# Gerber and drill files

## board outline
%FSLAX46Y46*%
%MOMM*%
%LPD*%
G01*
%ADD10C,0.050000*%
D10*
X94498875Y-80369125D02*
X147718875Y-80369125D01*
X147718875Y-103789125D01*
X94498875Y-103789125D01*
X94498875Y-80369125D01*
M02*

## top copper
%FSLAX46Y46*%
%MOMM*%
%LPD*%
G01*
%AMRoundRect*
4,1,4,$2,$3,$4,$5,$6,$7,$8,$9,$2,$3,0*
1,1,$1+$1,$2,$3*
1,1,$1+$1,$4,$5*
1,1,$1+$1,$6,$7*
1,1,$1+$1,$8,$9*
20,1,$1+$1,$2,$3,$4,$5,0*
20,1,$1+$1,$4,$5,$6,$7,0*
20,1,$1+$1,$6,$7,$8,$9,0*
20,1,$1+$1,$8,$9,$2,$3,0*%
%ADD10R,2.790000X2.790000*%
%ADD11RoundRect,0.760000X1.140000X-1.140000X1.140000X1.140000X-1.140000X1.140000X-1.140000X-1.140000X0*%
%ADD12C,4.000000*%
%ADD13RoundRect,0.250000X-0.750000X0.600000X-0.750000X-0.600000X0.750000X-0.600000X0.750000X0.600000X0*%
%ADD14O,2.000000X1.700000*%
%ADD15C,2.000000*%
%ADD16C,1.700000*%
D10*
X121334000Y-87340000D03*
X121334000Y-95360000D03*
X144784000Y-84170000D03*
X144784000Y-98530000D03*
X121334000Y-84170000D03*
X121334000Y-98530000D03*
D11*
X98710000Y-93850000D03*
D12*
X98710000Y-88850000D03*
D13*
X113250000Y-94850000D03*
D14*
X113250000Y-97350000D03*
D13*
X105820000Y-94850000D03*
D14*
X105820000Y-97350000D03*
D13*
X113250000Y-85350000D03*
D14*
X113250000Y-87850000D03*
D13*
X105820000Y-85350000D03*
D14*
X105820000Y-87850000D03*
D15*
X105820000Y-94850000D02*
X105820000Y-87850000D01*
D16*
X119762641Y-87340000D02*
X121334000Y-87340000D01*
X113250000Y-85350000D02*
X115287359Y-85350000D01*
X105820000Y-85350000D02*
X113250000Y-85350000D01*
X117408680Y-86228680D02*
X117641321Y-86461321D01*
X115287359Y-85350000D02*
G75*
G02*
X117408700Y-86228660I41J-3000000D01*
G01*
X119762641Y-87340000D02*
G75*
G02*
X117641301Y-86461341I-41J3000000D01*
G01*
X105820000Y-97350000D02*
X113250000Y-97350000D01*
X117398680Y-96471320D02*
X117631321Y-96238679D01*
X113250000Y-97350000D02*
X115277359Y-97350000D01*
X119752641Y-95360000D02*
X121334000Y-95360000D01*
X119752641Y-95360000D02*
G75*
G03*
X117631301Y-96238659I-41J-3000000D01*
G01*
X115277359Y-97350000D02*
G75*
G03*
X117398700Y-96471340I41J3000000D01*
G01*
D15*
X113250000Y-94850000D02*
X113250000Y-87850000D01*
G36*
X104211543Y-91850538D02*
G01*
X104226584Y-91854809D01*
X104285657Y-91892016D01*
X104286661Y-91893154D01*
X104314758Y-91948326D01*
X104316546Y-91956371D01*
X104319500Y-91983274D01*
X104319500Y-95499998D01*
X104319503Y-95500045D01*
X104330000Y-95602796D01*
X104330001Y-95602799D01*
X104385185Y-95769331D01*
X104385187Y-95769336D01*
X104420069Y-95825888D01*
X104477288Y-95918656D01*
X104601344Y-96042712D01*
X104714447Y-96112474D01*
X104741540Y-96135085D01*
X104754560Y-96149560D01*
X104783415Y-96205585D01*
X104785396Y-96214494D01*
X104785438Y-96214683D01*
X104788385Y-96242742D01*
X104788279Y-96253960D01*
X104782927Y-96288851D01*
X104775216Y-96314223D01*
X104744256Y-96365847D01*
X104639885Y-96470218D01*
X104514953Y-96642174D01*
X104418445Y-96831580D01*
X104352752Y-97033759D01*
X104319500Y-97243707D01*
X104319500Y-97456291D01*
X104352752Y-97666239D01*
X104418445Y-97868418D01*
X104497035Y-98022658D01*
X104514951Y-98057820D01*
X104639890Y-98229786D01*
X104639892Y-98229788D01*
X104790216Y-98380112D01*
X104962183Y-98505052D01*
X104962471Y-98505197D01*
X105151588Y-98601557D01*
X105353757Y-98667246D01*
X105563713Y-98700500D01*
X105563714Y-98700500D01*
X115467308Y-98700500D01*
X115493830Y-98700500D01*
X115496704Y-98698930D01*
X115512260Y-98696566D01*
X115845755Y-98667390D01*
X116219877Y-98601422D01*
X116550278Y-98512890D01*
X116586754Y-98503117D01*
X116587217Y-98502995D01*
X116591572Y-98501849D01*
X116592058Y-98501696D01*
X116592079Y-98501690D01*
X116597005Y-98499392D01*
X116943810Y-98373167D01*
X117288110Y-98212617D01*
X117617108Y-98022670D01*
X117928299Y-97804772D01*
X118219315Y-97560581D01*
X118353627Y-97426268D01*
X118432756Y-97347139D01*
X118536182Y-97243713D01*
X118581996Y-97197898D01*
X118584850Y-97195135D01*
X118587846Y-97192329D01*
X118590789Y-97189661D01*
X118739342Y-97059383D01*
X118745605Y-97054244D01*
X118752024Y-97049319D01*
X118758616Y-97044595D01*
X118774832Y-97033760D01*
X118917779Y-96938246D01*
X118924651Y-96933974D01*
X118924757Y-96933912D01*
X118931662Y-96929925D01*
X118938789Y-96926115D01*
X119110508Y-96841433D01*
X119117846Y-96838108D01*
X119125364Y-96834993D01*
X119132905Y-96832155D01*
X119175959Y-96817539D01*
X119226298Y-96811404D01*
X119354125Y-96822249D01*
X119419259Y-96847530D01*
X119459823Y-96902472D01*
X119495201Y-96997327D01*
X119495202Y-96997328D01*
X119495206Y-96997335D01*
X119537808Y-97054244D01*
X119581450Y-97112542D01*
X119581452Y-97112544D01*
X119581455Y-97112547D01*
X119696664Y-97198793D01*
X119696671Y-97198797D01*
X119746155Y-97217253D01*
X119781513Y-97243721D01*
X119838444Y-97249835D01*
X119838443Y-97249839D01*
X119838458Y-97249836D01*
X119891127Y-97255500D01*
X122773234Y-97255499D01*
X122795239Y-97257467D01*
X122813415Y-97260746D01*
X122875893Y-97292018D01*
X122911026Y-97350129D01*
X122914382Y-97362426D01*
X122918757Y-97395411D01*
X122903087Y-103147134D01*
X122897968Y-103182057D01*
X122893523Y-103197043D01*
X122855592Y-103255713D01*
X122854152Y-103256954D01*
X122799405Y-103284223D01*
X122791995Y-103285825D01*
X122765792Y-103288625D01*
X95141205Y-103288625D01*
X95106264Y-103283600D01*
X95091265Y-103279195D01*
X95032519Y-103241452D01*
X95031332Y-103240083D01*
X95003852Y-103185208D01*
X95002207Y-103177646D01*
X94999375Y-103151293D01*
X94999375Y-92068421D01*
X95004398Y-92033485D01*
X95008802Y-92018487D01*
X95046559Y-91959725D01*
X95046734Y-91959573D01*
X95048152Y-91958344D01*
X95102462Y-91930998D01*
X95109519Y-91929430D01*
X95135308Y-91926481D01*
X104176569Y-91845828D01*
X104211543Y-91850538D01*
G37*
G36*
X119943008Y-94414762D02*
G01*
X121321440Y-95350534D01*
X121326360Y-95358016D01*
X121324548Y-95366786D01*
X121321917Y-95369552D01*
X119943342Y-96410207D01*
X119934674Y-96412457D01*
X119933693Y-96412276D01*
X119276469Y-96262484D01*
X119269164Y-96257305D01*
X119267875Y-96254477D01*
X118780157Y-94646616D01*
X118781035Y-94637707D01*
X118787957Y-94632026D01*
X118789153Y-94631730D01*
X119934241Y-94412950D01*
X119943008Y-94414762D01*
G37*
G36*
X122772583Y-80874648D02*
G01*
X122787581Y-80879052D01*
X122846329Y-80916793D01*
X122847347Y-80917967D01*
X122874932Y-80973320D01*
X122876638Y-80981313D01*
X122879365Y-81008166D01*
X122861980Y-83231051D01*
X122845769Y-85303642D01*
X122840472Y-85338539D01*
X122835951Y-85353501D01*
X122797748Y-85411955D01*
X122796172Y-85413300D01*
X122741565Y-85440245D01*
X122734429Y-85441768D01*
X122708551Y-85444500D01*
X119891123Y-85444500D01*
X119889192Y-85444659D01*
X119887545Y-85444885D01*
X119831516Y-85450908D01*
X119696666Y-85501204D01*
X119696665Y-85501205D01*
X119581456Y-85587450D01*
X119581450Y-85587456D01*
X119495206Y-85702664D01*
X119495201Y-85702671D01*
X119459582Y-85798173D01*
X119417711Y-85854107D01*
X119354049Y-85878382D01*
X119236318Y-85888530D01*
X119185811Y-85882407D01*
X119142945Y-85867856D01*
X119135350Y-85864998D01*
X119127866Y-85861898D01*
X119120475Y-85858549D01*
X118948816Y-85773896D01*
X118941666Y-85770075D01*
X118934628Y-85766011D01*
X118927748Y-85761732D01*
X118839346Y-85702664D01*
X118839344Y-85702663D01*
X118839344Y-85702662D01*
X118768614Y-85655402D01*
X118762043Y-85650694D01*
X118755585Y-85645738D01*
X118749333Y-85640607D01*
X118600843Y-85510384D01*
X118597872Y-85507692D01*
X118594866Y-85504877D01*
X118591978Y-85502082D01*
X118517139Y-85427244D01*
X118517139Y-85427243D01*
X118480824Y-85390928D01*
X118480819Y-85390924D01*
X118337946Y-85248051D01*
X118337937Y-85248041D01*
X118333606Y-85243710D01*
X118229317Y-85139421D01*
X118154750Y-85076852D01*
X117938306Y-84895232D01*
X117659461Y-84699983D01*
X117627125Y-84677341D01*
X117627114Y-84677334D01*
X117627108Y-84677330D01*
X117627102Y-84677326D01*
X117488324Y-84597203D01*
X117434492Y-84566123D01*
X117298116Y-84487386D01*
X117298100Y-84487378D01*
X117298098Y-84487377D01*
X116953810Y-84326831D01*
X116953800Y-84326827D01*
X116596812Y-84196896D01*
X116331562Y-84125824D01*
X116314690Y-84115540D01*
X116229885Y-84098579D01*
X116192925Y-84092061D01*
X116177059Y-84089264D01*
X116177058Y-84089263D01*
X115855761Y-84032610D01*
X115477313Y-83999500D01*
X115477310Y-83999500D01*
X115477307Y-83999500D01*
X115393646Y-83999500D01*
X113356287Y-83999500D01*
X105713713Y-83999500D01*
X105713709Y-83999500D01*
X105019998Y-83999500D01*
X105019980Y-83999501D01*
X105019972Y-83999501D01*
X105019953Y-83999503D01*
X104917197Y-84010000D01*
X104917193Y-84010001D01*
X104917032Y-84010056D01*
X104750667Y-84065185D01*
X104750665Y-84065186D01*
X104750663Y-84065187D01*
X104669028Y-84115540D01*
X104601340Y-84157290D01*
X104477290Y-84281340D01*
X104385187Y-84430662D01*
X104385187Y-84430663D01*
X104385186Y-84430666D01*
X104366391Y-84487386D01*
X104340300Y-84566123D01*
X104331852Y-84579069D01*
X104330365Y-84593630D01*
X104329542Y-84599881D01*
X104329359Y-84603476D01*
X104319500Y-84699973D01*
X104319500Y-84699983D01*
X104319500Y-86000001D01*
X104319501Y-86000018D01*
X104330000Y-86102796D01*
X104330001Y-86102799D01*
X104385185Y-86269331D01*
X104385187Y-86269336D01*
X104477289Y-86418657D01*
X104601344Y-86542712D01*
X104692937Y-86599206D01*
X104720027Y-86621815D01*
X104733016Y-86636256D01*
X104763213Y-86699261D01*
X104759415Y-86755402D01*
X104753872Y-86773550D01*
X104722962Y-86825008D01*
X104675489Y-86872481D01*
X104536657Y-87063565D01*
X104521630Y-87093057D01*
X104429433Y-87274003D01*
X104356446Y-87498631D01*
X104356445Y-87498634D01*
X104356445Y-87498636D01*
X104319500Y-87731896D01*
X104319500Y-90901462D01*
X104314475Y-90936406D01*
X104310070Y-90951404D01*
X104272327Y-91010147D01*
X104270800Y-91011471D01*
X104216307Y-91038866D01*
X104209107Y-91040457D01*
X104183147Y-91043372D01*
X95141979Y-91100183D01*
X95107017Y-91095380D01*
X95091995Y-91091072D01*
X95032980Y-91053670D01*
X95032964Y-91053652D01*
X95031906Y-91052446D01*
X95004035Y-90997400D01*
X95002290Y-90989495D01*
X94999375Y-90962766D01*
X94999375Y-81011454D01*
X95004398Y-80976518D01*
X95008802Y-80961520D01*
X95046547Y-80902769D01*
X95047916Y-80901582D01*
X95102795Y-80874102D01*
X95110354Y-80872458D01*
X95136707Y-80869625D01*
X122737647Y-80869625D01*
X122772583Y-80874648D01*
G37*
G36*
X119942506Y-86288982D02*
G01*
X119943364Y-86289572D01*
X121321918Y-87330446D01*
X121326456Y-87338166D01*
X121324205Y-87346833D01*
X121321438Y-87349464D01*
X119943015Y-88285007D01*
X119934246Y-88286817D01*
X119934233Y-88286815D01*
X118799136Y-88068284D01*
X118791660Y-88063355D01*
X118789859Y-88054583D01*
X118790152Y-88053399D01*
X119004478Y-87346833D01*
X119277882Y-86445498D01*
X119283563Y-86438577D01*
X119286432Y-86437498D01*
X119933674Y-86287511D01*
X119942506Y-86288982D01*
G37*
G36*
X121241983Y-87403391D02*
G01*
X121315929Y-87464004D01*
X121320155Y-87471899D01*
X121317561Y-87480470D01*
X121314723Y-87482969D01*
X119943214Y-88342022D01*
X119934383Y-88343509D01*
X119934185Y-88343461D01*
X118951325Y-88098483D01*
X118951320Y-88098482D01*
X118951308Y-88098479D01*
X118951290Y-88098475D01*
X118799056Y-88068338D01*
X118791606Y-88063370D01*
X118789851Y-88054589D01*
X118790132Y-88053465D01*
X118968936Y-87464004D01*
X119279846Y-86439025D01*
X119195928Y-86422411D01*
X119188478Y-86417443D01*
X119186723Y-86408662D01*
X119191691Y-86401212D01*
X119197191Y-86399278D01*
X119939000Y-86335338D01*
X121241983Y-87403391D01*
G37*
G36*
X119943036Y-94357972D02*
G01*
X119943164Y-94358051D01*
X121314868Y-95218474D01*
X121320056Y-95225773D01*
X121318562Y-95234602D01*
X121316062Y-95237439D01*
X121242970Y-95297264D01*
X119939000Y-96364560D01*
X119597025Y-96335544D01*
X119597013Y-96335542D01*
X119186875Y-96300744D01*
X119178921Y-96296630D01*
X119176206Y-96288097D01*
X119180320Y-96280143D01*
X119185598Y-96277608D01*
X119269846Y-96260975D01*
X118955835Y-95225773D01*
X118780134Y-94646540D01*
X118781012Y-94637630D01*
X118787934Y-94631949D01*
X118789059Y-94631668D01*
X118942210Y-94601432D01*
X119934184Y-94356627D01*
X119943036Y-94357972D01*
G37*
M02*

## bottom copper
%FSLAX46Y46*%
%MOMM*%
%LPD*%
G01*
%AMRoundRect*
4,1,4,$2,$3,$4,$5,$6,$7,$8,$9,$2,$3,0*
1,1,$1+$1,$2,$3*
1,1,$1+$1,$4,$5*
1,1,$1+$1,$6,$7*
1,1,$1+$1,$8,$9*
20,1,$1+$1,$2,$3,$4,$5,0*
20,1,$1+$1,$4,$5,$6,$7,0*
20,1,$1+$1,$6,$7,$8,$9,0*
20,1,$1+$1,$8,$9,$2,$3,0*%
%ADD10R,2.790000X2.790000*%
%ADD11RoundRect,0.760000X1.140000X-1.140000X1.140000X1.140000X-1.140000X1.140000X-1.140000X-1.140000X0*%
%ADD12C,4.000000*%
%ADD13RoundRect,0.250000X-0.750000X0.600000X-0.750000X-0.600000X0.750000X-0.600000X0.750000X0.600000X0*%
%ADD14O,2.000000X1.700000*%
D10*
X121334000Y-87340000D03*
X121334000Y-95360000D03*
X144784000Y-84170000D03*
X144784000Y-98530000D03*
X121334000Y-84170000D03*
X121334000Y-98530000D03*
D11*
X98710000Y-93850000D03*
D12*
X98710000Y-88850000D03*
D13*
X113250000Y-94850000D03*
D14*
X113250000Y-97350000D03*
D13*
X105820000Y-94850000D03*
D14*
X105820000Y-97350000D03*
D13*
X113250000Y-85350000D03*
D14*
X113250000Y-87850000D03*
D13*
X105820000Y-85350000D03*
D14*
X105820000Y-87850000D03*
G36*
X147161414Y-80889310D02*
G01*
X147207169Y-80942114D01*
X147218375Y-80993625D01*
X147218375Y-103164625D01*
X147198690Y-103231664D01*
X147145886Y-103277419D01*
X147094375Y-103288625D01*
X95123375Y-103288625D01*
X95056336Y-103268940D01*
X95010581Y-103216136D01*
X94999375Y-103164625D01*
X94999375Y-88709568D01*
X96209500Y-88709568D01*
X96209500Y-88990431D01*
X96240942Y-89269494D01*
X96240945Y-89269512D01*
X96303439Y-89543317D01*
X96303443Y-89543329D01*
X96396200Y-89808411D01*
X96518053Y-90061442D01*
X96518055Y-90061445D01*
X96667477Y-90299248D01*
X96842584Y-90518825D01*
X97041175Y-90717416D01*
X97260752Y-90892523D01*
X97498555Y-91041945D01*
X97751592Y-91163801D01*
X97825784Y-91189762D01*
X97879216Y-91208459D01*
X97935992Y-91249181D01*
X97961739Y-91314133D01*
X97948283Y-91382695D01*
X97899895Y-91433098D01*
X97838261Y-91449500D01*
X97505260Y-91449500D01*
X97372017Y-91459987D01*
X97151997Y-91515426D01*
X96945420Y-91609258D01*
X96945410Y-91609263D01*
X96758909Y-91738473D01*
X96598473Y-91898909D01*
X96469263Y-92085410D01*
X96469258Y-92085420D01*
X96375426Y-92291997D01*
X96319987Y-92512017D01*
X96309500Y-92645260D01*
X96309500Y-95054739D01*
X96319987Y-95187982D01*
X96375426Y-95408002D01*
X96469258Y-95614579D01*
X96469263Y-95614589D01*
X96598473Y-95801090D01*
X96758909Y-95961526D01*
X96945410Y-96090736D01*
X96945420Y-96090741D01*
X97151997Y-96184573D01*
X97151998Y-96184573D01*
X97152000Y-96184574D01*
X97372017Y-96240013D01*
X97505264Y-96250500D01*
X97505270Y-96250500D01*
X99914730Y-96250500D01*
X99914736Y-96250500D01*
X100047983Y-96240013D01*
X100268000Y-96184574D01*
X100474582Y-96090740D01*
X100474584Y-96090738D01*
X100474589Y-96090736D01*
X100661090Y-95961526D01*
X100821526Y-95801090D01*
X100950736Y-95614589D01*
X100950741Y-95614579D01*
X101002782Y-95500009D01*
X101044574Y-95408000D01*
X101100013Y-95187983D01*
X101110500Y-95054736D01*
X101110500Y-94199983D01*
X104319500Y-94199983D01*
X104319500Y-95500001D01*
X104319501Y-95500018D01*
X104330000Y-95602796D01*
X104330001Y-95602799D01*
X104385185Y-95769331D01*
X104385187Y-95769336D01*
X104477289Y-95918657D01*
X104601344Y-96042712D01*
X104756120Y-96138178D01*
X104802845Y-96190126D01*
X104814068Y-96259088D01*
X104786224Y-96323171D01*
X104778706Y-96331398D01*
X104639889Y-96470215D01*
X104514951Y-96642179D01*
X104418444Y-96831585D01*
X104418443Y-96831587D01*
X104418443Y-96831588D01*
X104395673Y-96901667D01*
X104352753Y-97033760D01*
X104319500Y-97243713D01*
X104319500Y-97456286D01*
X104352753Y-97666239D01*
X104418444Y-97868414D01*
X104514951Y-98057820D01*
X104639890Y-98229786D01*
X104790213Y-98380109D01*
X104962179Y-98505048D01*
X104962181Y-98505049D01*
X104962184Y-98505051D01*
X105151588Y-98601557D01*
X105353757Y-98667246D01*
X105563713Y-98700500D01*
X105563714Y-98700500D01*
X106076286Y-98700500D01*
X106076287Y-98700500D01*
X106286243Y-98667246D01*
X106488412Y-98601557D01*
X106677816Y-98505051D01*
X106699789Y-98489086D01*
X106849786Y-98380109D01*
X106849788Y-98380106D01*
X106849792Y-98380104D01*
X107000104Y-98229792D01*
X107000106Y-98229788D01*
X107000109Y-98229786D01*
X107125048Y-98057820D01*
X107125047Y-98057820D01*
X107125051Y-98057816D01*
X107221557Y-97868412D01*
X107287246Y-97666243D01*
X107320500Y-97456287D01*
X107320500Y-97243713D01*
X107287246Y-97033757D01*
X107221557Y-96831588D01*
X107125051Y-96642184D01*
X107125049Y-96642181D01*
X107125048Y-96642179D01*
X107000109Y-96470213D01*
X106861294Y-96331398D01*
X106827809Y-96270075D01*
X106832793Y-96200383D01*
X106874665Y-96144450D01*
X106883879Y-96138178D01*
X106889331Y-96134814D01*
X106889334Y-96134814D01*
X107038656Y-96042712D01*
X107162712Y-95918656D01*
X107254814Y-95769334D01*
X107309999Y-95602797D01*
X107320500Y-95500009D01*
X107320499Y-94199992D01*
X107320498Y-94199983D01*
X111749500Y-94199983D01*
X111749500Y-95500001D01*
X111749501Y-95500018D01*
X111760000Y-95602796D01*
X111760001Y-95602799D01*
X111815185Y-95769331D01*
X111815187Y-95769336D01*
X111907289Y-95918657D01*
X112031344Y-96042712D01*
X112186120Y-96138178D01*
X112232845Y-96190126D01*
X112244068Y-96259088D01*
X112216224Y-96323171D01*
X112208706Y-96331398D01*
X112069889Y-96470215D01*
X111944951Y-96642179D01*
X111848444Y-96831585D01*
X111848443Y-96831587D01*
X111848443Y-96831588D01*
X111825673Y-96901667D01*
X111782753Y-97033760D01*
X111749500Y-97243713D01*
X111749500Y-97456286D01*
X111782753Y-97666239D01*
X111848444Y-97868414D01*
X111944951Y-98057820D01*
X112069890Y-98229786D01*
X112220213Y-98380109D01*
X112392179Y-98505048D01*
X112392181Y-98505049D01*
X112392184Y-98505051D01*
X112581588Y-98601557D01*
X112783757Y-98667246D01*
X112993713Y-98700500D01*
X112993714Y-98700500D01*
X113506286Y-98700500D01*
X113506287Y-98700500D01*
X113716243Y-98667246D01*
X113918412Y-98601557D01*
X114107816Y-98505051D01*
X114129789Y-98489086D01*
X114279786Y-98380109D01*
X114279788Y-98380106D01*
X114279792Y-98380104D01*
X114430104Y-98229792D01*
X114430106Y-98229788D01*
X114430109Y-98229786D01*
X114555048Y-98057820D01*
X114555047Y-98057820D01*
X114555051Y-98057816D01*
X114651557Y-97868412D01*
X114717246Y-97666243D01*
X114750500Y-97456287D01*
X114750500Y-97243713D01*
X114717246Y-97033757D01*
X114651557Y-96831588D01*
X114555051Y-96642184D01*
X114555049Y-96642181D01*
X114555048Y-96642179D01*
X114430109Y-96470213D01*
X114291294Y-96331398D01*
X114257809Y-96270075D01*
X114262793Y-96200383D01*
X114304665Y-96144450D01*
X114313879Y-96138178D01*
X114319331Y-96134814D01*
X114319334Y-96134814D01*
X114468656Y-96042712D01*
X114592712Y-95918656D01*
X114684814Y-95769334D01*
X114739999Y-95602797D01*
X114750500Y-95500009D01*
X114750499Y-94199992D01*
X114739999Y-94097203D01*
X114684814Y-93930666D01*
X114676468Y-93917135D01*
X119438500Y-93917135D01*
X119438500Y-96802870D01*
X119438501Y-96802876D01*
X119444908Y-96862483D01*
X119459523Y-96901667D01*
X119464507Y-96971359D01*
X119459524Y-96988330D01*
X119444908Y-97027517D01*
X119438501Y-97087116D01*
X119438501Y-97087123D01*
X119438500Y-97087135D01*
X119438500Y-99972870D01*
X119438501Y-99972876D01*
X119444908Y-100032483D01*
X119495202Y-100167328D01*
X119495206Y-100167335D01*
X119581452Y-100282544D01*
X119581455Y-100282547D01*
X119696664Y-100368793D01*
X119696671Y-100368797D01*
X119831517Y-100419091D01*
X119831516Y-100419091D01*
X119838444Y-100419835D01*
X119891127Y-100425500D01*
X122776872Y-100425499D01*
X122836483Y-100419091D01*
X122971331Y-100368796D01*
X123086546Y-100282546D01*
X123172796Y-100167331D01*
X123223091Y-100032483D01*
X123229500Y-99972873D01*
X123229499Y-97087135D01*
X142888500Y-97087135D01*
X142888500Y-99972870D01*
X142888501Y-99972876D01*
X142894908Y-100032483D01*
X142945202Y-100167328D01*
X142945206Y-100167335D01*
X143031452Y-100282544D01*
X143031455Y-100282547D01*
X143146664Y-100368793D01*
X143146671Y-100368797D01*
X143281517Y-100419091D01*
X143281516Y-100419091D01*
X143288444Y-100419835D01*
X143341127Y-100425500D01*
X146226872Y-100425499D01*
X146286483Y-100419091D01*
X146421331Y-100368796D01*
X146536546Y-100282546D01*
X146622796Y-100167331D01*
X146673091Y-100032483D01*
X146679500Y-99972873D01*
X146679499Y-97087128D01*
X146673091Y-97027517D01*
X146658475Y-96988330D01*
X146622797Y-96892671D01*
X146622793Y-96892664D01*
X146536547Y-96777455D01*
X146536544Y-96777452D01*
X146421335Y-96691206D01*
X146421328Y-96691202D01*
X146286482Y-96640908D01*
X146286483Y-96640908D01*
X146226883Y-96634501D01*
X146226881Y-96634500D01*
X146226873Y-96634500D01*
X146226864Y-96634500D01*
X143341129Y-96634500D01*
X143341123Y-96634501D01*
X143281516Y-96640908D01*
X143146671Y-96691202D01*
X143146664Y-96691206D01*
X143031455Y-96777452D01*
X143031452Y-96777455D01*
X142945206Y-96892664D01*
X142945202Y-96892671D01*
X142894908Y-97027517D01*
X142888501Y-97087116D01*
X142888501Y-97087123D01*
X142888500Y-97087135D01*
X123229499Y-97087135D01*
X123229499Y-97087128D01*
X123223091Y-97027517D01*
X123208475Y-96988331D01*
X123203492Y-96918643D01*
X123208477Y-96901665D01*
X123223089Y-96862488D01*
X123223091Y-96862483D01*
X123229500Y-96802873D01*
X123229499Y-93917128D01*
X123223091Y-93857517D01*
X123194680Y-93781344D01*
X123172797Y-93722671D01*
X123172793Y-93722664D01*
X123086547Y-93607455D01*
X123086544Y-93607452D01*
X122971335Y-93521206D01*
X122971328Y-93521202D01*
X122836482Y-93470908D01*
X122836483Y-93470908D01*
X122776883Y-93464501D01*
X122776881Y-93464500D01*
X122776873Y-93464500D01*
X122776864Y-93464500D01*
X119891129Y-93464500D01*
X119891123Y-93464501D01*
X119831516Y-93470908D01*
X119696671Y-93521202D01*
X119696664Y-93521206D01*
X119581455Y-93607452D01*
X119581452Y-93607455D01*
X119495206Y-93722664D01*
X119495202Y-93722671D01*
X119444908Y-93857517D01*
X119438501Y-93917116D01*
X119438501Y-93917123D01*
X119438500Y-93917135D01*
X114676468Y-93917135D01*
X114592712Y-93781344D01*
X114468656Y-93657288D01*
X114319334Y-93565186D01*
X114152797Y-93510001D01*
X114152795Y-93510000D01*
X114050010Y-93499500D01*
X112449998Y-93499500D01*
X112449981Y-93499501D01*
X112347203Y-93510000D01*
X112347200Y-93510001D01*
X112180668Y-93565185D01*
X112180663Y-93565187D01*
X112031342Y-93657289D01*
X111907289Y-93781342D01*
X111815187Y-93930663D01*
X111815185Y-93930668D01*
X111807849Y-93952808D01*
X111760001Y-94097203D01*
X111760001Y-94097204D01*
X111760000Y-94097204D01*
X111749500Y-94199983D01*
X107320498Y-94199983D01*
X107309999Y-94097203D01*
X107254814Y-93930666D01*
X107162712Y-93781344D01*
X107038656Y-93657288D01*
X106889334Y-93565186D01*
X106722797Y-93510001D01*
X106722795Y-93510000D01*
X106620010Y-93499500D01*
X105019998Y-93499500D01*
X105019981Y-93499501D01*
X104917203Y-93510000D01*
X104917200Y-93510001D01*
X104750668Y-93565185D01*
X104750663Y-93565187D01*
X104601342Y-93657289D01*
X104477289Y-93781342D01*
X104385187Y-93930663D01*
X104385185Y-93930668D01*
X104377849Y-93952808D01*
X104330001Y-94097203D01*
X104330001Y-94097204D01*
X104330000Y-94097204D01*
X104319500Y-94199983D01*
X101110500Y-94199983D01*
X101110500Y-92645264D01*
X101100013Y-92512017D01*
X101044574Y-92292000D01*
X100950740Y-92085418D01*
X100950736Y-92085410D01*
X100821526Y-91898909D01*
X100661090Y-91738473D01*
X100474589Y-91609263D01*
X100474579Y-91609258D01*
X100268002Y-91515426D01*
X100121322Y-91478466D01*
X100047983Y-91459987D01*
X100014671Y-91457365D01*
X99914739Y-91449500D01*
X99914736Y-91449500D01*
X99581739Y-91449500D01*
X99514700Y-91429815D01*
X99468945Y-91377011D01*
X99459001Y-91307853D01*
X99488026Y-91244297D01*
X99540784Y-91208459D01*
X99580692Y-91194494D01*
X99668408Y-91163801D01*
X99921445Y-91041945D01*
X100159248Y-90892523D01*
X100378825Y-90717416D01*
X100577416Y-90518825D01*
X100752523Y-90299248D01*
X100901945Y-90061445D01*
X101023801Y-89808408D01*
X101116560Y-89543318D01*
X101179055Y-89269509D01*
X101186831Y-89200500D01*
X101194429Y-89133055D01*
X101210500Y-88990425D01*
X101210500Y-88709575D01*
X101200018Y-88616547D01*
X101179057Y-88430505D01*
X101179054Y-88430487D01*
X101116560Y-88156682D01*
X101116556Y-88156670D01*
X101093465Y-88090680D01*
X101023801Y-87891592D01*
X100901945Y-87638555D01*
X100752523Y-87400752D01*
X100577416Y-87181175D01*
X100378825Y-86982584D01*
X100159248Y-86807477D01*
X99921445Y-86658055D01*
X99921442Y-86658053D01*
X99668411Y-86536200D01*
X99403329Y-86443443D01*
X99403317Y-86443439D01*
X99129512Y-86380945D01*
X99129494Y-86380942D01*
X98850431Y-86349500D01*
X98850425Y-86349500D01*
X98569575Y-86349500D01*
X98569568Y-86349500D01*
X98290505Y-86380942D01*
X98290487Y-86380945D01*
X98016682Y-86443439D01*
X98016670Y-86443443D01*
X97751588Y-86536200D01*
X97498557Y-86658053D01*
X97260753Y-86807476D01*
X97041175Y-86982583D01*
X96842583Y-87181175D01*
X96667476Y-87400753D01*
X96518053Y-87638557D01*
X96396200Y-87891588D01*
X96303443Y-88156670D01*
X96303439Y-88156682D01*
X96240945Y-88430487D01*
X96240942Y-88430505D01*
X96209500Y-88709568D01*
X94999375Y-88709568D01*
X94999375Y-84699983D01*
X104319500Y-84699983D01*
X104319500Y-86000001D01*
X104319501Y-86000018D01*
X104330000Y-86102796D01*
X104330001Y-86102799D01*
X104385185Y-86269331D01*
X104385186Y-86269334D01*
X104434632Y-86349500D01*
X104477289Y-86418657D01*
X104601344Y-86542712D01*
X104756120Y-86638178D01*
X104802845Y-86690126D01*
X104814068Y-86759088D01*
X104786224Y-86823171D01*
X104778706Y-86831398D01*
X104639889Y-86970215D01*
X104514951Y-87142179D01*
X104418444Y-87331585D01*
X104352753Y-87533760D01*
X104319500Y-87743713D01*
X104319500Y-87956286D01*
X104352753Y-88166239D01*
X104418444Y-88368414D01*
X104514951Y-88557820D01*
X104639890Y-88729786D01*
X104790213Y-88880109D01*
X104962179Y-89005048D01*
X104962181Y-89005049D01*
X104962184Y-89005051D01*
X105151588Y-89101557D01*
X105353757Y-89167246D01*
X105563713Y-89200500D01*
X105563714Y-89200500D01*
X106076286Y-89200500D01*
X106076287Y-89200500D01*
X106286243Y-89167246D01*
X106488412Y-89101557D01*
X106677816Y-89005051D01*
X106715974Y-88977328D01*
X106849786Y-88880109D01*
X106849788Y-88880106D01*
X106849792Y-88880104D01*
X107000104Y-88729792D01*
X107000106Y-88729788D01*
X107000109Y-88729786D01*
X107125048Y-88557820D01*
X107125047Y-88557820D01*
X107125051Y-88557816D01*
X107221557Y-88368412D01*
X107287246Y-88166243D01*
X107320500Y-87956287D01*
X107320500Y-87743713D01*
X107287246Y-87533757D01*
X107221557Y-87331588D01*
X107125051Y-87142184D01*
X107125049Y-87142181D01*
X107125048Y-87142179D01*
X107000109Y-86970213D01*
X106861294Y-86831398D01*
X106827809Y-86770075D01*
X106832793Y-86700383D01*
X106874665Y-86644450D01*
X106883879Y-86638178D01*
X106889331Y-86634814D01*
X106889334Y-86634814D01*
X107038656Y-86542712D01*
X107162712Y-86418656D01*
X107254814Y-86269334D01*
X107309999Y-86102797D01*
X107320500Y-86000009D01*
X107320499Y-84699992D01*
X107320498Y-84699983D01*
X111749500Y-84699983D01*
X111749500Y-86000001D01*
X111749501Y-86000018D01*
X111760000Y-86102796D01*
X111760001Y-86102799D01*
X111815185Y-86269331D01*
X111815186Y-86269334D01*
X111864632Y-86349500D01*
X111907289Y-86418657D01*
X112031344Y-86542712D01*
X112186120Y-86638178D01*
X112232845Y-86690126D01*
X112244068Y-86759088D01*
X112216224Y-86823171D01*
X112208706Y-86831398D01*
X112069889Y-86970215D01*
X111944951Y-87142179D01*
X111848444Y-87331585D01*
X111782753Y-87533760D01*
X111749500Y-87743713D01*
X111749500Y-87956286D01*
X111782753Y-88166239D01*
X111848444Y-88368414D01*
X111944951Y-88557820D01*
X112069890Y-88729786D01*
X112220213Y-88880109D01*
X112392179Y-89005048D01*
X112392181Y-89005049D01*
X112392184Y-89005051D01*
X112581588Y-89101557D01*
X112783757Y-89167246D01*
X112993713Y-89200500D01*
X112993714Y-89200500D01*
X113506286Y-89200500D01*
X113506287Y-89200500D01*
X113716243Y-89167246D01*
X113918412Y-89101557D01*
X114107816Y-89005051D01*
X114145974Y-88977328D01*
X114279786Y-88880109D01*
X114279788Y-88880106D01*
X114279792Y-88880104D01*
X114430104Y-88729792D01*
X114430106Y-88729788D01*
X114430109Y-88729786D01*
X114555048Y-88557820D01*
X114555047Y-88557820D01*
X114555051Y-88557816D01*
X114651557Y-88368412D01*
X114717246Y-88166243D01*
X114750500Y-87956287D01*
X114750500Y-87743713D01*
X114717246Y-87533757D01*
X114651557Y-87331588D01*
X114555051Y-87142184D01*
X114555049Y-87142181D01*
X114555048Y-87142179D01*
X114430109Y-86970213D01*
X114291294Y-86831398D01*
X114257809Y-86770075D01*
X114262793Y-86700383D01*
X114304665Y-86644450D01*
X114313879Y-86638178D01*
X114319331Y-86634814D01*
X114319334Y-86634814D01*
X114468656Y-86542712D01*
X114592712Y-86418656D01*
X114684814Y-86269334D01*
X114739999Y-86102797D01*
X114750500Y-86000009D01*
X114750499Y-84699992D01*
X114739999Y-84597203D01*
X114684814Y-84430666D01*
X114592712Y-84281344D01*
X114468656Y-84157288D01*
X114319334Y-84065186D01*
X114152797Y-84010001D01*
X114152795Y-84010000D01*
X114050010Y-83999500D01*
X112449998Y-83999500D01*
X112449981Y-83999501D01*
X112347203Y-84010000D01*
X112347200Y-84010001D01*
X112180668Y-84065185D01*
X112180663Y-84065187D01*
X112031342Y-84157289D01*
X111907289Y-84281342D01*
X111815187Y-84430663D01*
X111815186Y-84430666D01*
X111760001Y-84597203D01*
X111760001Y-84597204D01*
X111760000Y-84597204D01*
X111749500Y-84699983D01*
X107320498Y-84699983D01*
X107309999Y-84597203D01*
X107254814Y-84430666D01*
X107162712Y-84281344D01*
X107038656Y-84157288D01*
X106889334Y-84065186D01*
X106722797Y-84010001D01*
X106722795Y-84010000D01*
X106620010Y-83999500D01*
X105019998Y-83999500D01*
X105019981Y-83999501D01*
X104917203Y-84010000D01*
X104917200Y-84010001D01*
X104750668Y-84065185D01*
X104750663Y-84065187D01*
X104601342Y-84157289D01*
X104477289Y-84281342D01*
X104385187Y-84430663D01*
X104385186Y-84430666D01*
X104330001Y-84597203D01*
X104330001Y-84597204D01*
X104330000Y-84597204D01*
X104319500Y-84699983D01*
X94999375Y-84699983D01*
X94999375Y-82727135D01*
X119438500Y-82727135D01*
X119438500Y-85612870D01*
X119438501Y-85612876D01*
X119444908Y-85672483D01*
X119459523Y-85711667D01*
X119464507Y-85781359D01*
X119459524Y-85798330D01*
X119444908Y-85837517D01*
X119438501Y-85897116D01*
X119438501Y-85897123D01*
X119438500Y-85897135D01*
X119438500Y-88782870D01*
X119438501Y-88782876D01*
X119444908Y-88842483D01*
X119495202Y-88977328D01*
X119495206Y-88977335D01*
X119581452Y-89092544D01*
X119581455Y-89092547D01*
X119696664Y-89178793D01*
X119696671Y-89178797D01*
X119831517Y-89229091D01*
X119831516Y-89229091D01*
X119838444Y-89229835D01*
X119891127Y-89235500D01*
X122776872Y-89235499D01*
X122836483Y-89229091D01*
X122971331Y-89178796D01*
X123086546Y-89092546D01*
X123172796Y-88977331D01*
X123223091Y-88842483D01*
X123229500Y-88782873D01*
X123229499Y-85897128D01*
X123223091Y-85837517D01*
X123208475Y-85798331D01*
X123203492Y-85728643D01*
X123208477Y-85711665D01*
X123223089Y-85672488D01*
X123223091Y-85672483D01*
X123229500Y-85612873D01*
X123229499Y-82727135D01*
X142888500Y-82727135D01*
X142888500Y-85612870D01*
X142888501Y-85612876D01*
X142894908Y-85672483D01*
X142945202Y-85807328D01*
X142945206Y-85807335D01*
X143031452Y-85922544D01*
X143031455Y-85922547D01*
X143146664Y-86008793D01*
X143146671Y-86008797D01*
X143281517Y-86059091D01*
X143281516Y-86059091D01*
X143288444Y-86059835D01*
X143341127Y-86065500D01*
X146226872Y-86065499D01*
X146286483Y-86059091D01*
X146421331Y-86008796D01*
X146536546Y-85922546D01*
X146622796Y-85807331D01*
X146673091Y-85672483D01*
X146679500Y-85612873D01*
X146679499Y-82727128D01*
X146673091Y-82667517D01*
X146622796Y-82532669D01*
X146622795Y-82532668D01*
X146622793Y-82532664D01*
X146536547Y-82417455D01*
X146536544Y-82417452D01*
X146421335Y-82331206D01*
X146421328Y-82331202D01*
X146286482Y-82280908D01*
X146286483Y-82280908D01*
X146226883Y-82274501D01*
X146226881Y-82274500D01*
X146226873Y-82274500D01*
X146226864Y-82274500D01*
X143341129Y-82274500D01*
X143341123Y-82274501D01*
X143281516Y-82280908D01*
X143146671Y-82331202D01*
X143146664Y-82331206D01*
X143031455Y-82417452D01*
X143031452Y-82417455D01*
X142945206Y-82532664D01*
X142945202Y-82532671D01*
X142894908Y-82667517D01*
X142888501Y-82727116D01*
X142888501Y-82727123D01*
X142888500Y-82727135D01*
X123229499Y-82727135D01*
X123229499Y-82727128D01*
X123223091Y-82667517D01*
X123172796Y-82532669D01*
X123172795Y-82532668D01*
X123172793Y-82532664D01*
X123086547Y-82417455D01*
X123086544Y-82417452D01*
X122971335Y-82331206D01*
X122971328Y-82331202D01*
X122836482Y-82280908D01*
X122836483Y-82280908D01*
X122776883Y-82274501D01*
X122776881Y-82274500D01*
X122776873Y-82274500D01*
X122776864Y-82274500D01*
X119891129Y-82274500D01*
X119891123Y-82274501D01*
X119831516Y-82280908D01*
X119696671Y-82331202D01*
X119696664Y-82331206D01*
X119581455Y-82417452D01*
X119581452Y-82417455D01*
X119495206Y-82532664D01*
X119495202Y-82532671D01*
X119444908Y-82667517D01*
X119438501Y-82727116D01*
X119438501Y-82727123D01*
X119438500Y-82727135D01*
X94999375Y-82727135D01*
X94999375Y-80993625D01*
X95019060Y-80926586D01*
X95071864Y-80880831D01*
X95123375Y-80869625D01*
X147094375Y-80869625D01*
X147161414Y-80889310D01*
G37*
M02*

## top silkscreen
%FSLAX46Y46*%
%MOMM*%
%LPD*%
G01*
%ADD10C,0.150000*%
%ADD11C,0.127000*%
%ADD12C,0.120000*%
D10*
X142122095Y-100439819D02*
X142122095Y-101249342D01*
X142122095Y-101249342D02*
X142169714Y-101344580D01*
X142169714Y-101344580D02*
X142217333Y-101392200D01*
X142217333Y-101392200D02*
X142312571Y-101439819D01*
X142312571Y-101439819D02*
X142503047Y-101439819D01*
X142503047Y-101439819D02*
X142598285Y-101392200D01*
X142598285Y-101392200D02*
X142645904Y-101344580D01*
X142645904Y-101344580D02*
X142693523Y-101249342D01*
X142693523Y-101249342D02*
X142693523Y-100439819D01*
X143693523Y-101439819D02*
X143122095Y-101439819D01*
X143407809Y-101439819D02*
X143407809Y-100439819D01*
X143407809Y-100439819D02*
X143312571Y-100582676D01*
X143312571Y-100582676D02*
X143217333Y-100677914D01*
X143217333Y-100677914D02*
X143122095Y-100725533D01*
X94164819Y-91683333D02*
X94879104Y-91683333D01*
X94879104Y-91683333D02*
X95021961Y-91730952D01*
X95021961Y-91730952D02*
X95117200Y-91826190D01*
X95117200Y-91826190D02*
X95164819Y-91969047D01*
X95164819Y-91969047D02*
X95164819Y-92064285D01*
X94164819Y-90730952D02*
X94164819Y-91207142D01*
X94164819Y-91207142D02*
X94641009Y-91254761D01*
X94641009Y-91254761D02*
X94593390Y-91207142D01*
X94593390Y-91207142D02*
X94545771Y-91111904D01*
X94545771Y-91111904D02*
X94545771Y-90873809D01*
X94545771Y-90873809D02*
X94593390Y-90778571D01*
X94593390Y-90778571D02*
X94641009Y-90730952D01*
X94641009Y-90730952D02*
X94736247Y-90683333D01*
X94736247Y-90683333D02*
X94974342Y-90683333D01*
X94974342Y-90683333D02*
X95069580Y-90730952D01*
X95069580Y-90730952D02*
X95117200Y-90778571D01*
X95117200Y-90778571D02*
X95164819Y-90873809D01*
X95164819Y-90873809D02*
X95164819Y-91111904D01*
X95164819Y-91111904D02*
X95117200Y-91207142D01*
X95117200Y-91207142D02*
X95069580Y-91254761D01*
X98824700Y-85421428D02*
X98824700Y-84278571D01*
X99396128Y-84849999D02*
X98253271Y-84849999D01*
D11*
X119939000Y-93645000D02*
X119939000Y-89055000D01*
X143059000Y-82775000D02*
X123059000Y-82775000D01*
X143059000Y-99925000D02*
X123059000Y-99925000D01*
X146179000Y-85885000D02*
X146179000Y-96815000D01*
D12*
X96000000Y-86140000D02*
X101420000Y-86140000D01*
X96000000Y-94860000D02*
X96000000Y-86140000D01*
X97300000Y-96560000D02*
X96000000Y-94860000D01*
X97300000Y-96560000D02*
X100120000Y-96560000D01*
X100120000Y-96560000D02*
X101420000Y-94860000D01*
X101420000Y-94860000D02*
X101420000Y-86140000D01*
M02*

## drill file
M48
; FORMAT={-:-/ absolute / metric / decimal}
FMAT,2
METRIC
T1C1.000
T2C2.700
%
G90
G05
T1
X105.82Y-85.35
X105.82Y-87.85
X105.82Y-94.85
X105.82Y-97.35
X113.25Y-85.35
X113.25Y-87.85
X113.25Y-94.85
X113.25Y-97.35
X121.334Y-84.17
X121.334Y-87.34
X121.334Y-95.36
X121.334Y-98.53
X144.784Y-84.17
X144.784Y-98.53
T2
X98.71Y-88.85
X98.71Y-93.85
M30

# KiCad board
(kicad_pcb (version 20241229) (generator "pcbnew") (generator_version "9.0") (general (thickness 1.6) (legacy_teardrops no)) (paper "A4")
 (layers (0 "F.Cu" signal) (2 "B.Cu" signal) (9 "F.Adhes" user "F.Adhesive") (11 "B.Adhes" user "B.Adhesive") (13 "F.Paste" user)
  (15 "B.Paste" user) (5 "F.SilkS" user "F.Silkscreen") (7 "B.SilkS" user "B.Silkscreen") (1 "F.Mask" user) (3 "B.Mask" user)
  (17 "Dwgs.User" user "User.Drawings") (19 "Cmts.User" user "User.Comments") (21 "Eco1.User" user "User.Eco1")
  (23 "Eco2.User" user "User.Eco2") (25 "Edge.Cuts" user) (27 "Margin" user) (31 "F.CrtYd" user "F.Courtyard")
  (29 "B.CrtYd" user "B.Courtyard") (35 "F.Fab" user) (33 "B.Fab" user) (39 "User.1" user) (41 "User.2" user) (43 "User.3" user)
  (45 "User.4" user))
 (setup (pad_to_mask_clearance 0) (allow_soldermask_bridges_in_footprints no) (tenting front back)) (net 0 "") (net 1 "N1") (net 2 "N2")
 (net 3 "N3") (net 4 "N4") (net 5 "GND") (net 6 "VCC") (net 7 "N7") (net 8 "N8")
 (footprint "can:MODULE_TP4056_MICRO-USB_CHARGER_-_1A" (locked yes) (layer "F.Cu") (at 133.059 91.35 180)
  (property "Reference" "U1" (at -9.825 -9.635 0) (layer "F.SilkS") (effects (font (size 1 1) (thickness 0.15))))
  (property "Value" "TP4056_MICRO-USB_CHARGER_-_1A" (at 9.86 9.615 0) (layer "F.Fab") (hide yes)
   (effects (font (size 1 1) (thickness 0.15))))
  (fp_line (start 13.12 -2.295) (end 13.12 2.295) (stroke (width 0.127) (type solid)) (layer "F.SilkS"))
  (fp_line (start -10 8.575) (end 10 8.575) (stroke (width 0.127) (type solid)) (layer "F.SilkS"))
  (fp_line (start -10 -8.575) (end 10 -8.575) (stroke (width 0.127) (type solid)) (layer "F.SilkS"))
  (fp_line (start -13.12 5.465) (end -13.12 -5.465) (stroke (width 0.127) (type solid)) (layer "F.SilkS"))
  (pad "BAT_N" thru_hole rect (at 11.725 4.01 180) (size 2.79 2.79) (drill 1) (layers "*.Cu" "*.Mask") (remove_unused_layers no)
   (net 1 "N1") (solder_mask_margin 0.102)
   (teardrops (best_length_ratio 0.5) (max_length 1) (best_width_ratio 1) (max_width 2) (curved_edges no) (filter_ratio 0.9) (enabled yes)
    (allow_two_segments yes) (prefer_zone_connections yes)))
  (pad "BAT_P" thru_hole rect (at 11.725 -4.01 180) (size 2.79 2.79) (drill 1) (layers "*.Cu" "*.Mask") (remove_unused_layers no)
   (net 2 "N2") (solder_mask_margin 0.102)
   (teardrops (best_length_ratio 0.5) (max_length 1) (best_width_ratio 1) (max_width 2) (curved_edges no) (filter_ratio 0.9) (enabled yes)
    (allow_two_segments yes) (prefer_zone_connections yes)))
  (pad "IN_N" thru_hole rect (at -11.725 7.18 180) (size 2.79 2.79) (drill 1) (layers "*.Cu" "*.Mask") (remove_unused_layers no)
   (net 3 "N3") (solder_mask_margin 0.102)
   (teardrops (best_length_ratio 0.5) (max_length 1) (best_width_ratio 1) (max_width 2) (curved_edges no) (filter_ratio 0.9) (enabled yes)
    (allow_two_segments yes) (prefer_zone_connections yes)))
  (pad "IN_P" thru_hole rect (at -11.725 -7.18 180) (size 2.79 2.79) (drill 1) (layers "*.Cu" "*.Mask") (remove_unused_layers no)
   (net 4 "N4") (solder_mask_margin 0.102)
   (teardrops (best_length_ratio 0.5) (max_length 1) (best_width_ratio 1) (max_width 2) (curved_edges no) (filter_ratio 0.9) (enabled yes)
    (allow_two_segments yes) (prefer_zone_connections yes)))
  (pad "OUT_N" thru_hole rect (at 11.725 7.18 180) (size 2.79 2.79) (drill 1) (layers "*.Cu" "*.Mask") (remove_unused_layers no)
   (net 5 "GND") (solder_mask_margin 0.102)
   (teardrops (best_length_ratio 0.5) (max_length 1) (best_width_ratio 1) (max_width 2) (curved_edges no) (filter_ratio 0.9) (enabled yes)
    (allow_two_segments yes) (prefer_zone_connections yes)))
  (pad "OUT_P" thru_hole rect (at 11.725 -7.18 180) (size 2.79 2.79) (drill 1) (layers "*.Cu" "*.Mask") (remove_unused_layers no)
   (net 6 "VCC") (solder_mask_margin 0.102)
   (teardrops (best_length_ratio 0.5) (max_length 1) (best_width_ratio 1) (max_width 2) (curved_edges no) (filter_ratio 0.9) (enabled yes)
    (allow_two_segments yes) (prefer_zone_connections yes))))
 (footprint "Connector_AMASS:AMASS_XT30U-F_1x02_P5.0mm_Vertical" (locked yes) (layer "F.Cu") (at 98.71 93.85 90)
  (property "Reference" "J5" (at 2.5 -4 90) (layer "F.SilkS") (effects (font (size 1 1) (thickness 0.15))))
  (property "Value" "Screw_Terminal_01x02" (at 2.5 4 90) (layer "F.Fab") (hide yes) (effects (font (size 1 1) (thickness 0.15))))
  (fp_line (start 7.71 -2.71) (end 7.71 2.71) (stroke (width 0.12) (type solid)) (layer "F.SilkS"))
  (fp_line (start -1.01 -2.71) (end 7.71 -2.71) (stroke (width 0.12) (type solid)) (layer "F.SilkS"))
  (fp_line (start -2.71 -1.41) (end -1.01 -2.71) (stroke (width 0.12) (type solid)) (layer "F.SilkS"))
  (fp_line (start -2.71 -1.41) (end -2.71 1.41) (stroke (width 0.12) (type solid)) (layer "F.SilkS"))
  (fp_line (start -2.71 1.41) (end -1.01 2.71) (stroke (width 0.12) (type solid)) (layer "F.SilkS"))
  (fp_line (start -1.01 2.71) (end 7.71 2.71) (stroke (width 0.12) (type solid)) (layer "F.SilkS"))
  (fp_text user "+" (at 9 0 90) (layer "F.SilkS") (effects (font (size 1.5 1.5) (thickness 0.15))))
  (pad "1" thru_hole roundrect (at 0 0 90) (size 3.8 3.8) (drill 2.7) (layers "*.Cu" "*.Mask") (remove_unused_layers no)
   (roundrect_rratio 0.2) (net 6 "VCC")
   (teardrops (best_length_ratio 0.5) (max_length 1) (best_width_ratio 1) (max_width 2) (curved_edges no) (filter_ratio 0.9) (enabled yes)
    (allow_two_segments yes) (prefer_zone_connections yes)))
  (pad "2" thru_hole circle (at 5 0 90) (size 4 4) (drill 2.7) (layers "*.Cu" "*.Mask") (remove_unused_layers no) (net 5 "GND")
   (teardrops (best_length_ratio 0.5) (max_length 1) (best_width_ratio 1) (max_width 2) (curved_edges no) (filter_ratio 0.9) (enabled yes)
    (allow_two_segments yes) (prefer_zone_connections yes))))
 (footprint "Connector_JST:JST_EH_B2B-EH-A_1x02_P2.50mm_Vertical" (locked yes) (layer "B.Cu") (at 113.25 94.85 -90)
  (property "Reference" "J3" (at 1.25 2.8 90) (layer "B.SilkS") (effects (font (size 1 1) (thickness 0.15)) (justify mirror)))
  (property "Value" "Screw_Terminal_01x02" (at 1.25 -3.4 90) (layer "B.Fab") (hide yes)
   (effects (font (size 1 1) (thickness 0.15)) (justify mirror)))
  (pad "1" thru_hole roundrect (at 0 0 270) (size 1.7 2) (drill 1) (layers "*.Cu" "*.Mask") (remove_unused_layers no)
   (roundrect_rratio 0.147059) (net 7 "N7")
   (teardrops (best_length_ratio 0.5) (max_length 1) (best_width_ratio 1) (max_width 2) (curved_edges no) (filter_ratio 0.9) (enabled yes)
    (allow_two_segments yes) (prefer_zone_connections yes)))
  (pad "2" thru_hole oval (at 2.5 0 270) (size 1.7 2) (drill 1) (layers "*.Cu" "*.Mask") (remove_unused_layers no) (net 2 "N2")
   (teardrops (best_length_ratio 0.5) (max_length 1) (best_width_ratio 1) (max_width 2) (curved_edges no) (filter_ratio 0.9) (enabled yes)
    (allow_two_segments yes) (prefer_zone_connections yes))))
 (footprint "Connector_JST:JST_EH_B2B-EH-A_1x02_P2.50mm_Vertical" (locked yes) (layer "B.Cu") (at 105.82 94.85 -90)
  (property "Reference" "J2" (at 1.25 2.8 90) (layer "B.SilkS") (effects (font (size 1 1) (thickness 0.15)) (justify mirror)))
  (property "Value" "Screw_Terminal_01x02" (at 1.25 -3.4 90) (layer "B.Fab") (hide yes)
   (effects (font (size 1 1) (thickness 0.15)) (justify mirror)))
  (pad "1" thru_hole roundrect (at 0 0 270) (size 1.7 2) (drill 1) (layers "*.Cu" "*.Mask") (remove_unused_layers no)
   (roundrect_rratio 0.147059) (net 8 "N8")
   (teardrops (best_length_ratio 0.5) (max_length 1) (best_width_ratio 1) (max_width 2) (curved_edges no) (filter_ratio 0.9) (enabled yes)
    (allow_two_segments yes) (prefer_zone_connections yes)))
  (pad "2" thru_hole oval (at 2.5 0 270) (size 1.7 2) (drill 1) (layers "*.Cu" "*.Mask") (remove_unused_layers no) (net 2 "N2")
   (teardrops (best_length_ratio 0.5) (max_length 1) (best_width_ratio 1) (max_width 2) (curved_edges no) (filter_ratio 0.9) (enabled yes)
    (allow_two_segments yes) (prefer_zone_connections yes))))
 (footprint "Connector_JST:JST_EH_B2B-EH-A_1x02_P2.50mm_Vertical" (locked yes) (layer "B.Cu") (at 113.25 85.35 -90)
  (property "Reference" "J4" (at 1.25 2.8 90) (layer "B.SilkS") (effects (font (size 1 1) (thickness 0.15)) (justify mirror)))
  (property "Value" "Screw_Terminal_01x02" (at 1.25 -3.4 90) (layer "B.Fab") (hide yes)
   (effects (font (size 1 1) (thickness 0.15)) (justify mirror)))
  (pad "1" thru_hole roundrect (at 0 0 270) (size 1.7 2) (drill 1) (layers "*.Cu" "*.Mask") (remove_unused_layers no)
   (roundrect_rratio 0.147059) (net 1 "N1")
   (teardrops (best_length_ratio 0.5) (max_length 1) (best_width_ratio 1) (max_width 2) (curved_edges no) (filter_ratio 0.9) (enabled yes)
    (allow_two_segments yes) (prefer_zone_connections yes)))
  (pad "2" thru_hole oval (at 2.5 0 270) (size 1.7 2) (drill 1) (layers "*.Cu" "*.Mask") (remove_unused_layers no) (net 7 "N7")
   (teardrops (best_length_ratio 0.5) (max_length 1) (best_width_ratio 1) (max_width 2) (curved_edges no) (filter_ratio 0.9) (enabled yes)
    (allow_two_segments yes) (prefer_zone_connections yes))))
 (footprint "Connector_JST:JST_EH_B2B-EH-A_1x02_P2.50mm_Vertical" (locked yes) (layer "B.Cu") (at 105.82 85.35 -90)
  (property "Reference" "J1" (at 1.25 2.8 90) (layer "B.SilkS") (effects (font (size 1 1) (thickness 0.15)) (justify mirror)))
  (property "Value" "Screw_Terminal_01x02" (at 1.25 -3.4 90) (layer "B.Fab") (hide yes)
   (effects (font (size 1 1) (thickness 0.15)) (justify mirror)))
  (pad "1" thru_hole roundrect (at 0 0 270) (size 1.7 2) (drill 1) (layers "*.Cu" "*.Mask") (remove_unused_layers no)
   (roundrect_rratio 0.147059) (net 1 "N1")
   (teardrops (best_length_ratio 0.5) (max_length 1) (best_width_ratio 1) (max_width 2) (curved_edges no) (filter_ratio 0.9) (enabled yes)
    (allow_two_segments yes) (prefer_zone_connections yes)))
  (pad "2" thru_hole oval (at 2.5 0 270) (size 1.7 2) (drill 1) (layers "*.Cu" "*.Mask") (remove_unused_layers no) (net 8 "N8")
   (teardrops (best_length_ratio 0.5) (max_length 1) (best_width_ratio 1) (max_width 2) (curved_edges no) (filter_ratio 0.9) (enabled yes)
    (allow_two_segments yes) (prefer_zone_connections yes))))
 (gr_rect (start 94.498875 80.369125) (end 147.718875 103.789125) (stroke (width 0.05) (type default)) (fill no) (layer "Edge.Cuts"))
 (segment (start 105.82 94.85) (end 105.82 87.85) (width 2) (locked yes) (layer "F.Cu") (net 8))
 (segment (start 119.762641 87.34) (end 121.334 87.34) (width 1.7) (locked yes) (layer "F.Cu") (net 1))
 (segment (start 113.25 85.35) (end 115.287359 85.35) (width 1.7) (locked yes) (layer "F.Cu") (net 1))
 (segment (start 105.82 85.35) (end 113.25 85.35) (width 1.7) (locked yes) (layer "F.Cu") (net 1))
 (segment (start 117.40868 86.22868) (end 117.641321 86.461321) (width 1.7) (locked yes) (layer "F.Cu") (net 1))
 (arc (start 115.287359 85.35) (mid 116.43541 85.578362) (end 117.40868 86.22868) (width 1.7) (locked yes) (layer "F.Cu") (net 1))
 (arc (start 119.762641 87.34) (mid 118.614591 87.111639) (end 117.641321 86.461321) (width 1.7) (locked yes) (layer "F.Cu") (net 1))
 (segment (start 105.82 97.35) (end 113.25 97.35) (width 1.7) (locked yes) (layer "F.Cu") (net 2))
 (segment (start 117.39868 96.47132) (end 117.631321 96.238679) (width 1.7) (locked yes) (layer "F.Cu") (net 2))
 (segment (start 113.25 97.35) (end 115.277359 97.35) (width 1.7) (locked yes) (layer "F.Cu") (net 2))
 (segment (start 119.752641 95.36) (end 121.334 95.36) (width 1.7) (locked yes) (layer "F.Cu") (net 2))
 (arc (start 119.752641 95.36) (mid 118.604591 95.588361) (end 117.631321 96.238679) (width 1.7) (locked yes) (layer "F.Cu") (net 2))
 (arc (start 115.277359 97.35) (mid 116.42541 97.121638) (end 117.39868 96.47132) (width 1.7) (locked yes) (layer "F.Cu") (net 2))
 (segment (start 113.25 94.85) (end 113.25 87.85) (width 2) (locked yes) (layer "F.Cu") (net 7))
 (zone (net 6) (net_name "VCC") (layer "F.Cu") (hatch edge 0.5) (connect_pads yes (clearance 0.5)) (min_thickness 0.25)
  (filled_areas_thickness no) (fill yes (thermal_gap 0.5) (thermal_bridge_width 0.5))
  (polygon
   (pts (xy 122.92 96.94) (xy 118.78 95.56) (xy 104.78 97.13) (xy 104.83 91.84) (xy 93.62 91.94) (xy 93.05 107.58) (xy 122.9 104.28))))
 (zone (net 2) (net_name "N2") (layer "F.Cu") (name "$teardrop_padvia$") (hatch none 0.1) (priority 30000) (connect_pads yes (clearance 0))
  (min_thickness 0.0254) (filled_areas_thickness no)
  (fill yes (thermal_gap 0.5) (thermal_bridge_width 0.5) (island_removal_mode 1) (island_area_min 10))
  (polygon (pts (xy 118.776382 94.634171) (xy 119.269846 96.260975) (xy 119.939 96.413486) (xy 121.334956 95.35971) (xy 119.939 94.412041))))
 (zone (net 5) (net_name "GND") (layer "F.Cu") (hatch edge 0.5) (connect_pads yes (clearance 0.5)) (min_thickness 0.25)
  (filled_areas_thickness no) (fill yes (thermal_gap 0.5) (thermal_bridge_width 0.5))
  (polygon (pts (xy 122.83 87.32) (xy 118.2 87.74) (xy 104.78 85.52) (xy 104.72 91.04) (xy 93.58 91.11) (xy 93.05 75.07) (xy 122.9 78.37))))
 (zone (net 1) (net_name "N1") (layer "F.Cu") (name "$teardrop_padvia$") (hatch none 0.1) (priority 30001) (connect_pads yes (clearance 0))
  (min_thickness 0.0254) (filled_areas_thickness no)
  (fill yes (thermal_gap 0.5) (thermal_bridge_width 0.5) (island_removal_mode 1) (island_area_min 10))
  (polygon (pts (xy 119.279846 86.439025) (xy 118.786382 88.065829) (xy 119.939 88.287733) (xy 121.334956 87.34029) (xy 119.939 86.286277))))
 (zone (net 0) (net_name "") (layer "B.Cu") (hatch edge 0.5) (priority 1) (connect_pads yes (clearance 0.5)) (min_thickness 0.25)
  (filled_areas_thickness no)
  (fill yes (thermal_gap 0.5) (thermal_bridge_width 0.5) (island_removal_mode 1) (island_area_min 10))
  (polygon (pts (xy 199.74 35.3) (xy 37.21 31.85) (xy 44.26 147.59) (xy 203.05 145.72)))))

